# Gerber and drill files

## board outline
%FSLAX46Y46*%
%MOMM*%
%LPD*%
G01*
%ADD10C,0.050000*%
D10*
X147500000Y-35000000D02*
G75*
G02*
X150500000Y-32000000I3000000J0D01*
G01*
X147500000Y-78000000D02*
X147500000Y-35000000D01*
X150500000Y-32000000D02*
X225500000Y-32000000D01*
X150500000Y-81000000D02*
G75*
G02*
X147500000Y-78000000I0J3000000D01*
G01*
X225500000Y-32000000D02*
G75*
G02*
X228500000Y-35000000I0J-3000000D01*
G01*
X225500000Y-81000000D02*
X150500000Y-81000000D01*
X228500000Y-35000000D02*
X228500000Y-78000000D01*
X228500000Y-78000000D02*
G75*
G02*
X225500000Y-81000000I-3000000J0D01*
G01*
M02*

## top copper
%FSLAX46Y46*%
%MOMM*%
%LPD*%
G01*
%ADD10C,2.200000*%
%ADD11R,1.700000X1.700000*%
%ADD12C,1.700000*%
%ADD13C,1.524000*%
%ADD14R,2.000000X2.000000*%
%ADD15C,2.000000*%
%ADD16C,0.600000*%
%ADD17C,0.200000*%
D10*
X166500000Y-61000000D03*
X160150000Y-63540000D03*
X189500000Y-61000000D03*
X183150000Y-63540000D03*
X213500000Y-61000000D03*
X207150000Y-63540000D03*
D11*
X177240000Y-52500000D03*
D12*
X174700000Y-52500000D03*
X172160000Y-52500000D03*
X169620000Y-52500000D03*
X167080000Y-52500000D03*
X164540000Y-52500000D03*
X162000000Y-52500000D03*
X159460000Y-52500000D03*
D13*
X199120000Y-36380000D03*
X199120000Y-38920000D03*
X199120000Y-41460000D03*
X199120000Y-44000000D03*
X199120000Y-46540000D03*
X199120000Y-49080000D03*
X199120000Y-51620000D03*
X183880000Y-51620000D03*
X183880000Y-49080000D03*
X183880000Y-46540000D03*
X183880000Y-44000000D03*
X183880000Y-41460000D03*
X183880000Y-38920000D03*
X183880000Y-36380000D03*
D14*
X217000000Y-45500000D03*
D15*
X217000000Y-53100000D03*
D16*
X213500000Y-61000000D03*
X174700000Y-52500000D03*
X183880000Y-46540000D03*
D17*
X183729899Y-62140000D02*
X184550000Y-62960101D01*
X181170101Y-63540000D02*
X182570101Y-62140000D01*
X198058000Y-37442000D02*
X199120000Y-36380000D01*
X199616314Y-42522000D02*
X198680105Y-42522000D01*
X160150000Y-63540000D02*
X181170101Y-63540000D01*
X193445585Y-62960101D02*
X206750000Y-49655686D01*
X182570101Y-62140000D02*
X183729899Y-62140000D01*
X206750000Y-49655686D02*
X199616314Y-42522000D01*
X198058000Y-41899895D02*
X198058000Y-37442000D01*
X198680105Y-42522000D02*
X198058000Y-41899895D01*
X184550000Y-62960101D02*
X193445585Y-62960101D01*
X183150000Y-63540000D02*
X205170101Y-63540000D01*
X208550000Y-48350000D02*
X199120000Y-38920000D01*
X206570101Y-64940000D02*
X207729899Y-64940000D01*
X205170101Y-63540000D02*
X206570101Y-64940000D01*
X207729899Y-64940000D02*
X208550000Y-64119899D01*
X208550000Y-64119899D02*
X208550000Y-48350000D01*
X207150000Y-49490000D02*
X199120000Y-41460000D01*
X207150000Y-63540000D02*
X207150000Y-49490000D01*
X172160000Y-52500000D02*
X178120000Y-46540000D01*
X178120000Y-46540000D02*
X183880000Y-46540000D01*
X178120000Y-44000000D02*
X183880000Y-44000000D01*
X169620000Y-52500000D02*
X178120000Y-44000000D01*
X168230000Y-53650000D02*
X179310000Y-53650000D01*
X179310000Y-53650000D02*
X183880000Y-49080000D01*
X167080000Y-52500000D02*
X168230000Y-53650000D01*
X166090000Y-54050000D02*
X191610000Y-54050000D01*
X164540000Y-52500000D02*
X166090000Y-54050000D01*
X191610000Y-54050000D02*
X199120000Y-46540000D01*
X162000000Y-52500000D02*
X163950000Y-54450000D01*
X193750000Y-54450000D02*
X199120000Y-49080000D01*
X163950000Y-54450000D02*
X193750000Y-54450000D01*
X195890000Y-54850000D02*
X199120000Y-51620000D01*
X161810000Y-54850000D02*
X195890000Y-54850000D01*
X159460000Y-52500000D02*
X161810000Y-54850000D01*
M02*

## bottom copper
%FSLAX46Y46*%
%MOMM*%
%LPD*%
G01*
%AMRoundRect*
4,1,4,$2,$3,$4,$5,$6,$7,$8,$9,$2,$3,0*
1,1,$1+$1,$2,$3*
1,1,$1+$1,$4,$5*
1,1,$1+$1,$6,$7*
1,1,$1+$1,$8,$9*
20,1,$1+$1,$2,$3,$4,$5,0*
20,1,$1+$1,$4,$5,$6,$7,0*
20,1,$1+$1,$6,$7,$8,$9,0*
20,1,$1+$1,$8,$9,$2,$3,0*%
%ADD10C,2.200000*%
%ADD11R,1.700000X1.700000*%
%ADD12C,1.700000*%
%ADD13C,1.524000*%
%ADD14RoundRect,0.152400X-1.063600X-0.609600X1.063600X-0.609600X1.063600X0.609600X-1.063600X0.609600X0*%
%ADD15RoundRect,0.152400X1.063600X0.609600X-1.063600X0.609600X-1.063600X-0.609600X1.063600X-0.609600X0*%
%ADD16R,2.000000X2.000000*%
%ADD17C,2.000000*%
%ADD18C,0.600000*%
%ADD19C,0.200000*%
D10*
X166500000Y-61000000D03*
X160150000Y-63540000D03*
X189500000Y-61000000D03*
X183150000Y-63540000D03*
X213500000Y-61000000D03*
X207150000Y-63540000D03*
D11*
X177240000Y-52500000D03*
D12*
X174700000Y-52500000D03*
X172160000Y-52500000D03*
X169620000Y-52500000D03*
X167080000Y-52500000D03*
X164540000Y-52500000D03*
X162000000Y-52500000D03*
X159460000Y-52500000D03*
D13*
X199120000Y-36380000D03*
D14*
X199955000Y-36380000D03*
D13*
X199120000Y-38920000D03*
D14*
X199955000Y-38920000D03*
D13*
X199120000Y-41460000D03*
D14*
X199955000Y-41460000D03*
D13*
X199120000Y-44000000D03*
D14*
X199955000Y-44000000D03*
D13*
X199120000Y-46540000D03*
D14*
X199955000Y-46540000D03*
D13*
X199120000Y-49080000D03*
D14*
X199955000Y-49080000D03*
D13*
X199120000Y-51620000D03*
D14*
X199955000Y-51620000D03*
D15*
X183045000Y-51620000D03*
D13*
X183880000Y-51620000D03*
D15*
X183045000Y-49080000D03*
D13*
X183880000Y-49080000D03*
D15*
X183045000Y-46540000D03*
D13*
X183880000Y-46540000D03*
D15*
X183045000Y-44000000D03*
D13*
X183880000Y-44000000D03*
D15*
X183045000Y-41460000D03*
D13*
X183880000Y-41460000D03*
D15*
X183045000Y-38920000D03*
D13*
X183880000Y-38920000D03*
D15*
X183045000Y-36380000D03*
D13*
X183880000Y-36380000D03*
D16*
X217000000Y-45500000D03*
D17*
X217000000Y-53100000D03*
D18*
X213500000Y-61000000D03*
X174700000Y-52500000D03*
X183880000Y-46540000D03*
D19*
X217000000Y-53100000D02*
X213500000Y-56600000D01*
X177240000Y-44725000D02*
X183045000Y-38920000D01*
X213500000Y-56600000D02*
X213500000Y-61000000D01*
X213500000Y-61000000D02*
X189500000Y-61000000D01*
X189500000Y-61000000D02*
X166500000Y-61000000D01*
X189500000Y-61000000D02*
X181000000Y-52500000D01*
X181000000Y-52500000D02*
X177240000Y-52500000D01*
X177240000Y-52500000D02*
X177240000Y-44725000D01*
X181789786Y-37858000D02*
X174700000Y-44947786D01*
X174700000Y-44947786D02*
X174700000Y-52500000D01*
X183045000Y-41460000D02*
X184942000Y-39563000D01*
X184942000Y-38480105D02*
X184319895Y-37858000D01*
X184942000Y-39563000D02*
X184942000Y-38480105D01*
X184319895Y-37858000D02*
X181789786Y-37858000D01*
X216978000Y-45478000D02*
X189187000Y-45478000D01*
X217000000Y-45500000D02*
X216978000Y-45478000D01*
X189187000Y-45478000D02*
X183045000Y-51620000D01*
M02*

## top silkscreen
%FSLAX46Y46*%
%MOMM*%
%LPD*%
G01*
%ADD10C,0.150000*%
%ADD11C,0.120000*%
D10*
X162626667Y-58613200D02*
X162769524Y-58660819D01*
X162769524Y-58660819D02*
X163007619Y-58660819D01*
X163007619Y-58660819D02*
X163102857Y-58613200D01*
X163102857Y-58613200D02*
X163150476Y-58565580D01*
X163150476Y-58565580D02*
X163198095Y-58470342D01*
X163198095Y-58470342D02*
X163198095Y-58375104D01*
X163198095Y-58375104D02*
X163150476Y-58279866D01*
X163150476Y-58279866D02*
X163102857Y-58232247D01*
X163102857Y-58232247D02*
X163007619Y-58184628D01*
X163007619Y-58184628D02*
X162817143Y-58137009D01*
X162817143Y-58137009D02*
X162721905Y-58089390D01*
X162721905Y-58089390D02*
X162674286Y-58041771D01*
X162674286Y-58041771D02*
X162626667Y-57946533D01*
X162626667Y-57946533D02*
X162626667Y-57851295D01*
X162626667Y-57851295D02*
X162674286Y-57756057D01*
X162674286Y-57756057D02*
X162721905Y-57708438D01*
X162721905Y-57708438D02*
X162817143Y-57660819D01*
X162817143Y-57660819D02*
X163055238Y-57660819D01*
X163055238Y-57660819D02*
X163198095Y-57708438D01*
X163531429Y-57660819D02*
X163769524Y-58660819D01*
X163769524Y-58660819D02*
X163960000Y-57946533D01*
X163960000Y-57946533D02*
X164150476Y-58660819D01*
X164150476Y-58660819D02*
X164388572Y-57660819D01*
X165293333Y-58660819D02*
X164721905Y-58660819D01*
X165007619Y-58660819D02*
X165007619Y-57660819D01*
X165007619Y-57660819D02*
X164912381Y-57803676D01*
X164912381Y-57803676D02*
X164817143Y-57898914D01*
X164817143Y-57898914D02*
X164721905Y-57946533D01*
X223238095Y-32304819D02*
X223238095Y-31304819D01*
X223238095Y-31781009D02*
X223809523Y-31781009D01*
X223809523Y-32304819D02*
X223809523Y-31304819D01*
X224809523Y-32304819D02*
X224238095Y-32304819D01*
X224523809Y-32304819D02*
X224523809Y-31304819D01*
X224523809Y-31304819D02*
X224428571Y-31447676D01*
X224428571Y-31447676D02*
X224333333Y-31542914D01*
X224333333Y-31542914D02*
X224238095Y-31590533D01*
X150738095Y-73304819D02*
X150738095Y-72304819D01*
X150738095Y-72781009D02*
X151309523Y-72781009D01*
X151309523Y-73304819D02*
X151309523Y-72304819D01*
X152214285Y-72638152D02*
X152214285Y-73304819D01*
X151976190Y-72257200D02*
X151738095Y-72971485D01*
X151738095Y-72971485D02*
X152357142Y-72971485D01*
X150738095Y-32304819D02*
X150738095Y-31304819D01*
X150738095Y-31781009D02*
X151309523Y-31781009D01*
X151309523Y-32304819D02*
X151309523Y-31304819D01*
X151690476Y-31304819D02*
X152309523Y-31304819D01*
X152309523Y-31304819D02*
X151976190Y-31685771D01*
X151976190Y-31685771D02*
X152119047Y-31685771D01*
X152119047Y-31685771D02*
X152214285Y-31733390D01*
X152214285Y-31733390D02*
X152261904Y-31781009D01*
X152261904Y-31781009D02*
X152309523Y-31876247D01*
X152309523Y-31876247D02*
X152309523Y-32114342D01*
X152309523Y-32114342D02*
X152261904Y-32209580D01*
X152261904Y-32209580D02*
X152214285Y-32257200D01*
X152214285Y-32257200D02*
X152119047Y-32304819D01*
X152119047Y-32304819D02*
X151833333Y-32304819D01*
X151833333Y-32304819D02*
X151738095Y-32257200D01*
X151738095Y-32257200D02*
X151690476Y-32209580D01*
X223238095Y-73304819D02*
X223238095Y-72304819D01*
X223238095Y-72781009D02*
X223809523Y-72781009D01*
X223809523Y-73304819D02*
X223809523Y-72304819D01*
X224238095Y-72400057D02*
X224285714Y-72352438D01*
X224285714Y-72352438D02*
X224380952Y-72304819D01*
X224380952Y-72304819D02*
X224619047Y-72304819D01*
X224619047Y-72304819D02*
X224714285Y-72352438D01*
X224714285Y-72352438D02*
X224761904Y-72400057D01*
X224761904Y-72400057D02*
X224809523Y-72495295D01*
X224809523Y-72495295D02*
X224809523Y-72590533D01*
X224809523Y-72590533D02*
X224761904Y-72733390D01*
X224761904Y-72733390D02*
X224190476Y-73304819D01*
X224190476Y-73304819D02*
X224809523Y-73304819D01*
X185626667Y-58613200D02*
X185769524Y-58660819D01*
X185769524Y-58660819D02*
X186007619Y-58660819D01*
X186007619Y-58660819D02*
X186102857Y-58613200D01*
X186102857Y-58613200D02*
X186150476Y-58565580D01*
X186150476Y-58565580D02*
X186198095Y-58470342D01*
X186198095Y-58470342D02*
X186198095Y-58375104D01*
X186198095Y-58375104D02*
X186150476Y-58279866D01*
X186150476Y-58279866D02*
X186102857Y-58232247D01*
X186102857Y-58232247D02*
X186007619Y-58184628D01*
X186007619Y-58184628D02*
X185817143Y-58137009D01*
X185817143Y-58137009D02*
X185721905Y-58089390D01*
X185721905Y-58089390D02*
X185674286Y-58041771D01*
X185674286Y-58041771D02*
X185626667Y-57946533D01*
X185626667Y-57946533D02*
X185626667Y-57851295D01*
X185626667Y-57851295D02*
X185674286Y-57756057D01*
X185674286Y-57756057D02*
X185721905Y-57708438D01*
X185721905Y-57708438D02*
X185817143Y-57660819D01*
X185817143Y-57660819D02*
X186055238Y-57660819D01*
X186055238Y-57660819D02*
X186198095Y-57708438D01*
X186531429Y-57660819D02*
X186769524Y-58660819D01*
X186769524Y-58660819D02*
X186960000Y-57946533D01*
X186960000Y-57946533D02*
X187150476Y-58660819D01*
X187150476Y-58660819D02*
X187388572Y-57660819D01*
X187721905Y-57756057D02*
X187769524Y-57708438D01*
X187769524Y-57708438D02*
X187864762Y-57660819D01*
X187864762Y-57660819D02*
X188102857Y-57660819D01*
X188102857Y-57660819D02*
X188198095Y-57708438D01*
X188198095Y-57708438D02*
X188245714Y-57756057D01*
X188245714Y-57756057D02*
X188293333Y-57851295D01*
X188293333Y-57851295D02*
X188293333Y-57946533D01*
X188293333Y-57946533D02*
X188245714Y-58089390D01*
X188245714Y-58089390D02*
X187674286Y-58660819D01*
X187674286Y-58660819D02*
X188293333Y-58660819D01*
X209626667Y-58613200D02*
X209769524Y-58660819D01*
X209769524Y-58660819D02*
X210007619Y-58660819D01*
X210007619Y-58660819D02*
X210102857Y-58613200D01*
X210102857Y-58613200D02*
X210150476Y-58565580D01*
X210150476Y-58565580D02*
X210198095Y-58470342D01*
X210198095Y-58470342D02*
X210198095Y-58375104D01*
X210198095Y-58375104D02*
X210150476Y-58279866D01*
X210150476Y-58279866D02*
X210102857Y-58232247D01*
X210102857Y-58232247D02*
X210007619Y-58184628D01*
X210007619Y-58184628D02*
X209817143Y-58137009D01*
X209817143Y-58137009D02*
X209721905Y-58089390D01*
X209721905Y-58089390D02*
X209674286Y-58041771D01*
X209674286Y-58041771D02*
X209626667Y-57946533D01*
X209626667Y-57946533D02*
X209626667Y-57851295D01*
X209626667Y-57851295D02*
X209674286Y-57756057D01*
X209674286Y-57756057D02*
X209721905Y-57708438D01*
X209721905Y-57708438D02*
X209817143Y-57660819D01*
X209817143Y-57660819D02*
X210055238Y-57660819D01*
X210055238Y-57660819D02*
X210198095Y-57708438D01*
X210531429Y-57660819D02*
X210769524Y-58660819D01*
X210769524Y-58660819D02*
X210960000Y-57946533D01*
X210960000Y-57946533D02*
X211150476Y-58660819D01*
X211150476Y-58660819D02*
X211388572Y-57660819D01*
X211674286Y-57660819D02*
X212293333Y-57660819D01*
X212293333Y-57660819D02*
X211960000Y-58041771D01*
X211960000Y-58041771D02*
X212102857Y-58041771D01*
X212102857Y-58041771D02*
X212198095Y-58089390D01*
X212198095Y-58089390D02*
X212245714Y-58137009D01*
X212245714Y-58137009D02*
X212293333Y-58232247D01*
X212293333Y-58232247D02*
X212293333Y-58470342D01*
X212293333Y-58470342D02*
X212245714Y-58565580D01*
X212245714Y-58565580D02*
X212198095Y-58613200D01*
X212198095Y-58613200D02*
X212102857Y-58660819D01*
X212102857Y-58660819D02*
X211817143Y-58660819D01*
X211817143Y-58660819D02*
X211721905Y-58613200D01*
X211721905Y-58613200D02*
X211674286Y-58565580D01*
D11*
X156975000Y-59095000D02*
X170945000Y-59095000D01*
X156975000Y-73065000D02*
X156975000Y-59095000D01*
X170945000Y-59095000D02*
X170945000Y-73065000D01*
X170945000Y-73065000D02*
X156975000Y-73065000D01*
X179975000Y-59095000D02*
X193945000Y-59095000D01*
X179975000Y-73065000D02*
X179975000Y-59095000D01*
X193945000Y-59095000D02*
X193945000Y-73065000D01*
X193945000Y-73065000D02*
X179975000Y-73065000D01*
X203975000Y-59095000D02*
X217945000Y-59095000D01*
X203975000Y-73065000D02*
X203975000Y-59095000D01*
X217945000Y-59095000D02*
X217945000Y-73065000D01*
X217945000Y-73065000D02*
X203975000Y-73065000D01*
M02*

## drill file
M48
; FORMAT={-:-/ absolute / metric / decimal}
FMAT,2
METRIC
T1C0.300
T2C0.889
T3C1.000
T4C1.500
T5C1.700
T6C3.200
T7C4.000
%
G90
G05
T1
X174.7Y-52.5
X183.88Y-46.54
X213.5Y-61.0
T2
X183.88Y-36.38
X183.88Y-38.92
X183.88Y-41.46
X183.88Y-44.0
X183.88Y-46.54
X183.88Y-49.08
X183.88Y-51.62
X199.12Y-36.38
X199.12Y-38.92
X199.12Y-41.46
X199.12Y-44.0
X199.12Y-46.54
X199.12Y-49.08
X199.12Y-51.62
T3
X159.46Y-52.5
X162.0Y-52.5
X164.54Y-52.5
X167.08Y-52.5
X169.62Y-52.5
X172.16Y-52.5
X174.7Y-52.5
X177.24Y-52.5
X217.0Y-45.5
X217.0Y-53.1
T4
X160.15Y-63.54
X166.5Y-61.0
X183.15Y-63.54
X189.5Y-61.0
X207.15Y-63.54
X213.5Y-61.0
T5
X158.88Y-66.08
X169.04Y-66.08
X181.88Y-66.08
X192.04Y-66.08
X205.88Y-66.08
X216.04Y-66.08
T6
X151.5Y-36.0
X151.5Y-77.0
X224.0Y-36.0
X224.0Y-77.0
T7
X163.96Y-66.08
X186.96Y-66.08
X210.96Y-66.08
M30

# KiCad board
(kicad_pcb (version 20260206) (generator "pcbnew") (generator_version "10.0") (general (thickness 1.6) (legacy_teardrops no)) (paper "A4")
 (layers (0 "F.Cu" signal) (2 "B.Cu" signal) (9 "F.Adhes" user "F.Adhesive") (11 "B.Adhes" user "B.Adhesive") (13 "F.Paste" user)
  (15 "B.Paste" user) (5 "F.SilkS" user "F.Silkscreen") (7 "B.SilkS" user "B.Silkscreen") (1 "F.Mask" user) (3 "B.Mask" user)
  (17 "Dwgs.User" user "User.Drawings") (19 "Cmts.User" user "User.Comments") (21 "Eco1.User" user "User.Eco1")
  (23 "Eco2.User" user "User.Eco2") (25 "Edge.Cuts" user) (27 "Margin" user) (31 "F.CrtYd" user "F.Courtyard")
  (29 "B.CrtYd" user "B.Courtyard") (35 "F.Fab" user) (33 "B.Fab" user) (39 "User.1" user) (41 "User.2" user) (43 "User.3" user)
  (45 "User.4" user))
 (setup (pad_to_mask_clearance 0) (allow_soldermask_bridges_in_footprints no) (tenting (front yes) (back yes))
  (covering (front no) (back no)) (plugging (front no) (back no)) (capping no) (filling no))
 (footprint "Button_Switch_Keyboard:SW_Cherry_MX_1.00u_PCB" (layer "F.Cu") (at 166.5 61)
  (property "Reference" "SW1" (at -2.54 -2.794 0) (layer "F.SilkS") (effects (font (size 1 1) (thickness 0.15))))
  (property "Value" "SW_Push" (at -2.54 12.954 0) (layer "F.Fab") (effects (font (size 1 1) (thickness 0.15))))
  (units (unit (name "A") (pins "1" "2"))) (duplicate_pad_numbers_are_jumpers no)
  (fp_line (start -9.525 -1.905) (end 4.445 -1.905) (stroke (width 0.12) (type solid)) (layer "F.SilkS"))
  (fp_line (start -9.525 12.065) (end -9.525 -1.905) (stroke (width 0.12) (type solid)) (layer "F.SilkS"))
  (fp_line (start 4.445 -1.905) (end 4.445 12.065) (stroke (width 0.12) (type solid)) (layer "F.SilkS"))
  (fp_line (start 4.445 12.065) (end -9.525 12.065) (stroke (width 0.12) (type solid)) (layer "F.SilkS"))
  (pad "" np_thru_hole circle (at -7.62 5.08) (size 1.7 1.7) (drill 1.7) (layers "*.Cu" "*.Mask"))
  (pad "" np_thru_hole circle (at -2.54 5.08) (size 4 4) (drill 4) (layers "*.Cu" "*.Mask"))
  (pad "" np_thru_hole circle (at 2.54 5.08) (size 1.7 1.7) (drill 1.7) (layers "*.Cu" "*.Mask"))
  (pad "1" thru_hole circle (at 0 0) (size 2.2 2.2) (drill 1.5) (layers "*.Cu" "*.Mask") (remove_unused_layers no) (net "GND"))
  (pad "2" thru_hole circle (at -6.35 2.54) (size 2.2 2.2) (drill 1.5) (layers "*.Cu" "*.Mask") (remove_unused_layers no)
   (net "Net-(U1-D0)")))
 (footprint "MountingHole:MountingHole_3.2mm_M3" (layer "F.Cu") (at 224 36)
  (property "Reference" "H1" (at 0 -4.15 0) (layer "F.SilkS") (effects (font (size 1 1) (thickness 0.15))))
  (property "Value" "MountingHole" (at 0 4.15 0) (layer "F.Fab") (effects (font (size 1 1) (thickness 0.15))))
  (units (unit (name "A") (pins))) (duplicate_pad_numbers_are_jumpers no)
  (pad "" np_thru_hole circle (at 0 0) (size 3.2 3.2) (drill 3.2) (layers "*.Cu" "*.Mask")))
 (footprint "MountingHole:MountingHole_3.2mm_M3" (layer "F.Cu") (at 151.5 77)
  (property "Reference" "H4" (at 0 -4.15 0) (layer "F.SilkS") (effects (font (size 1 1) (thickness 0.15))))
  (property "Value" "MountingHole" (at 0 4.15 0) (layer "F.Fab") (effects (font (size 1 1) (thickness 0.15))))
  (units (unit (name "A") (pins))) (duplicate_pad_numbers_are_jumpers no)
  (pad "" np_thru_hole circle (at 0 0) (size 3.2 3.2) (drill 3.2) (layers "*.Cu" "*.Mask")))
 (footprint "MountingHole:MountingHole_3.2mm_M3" (layer "F.Cu") (at 151.5 36)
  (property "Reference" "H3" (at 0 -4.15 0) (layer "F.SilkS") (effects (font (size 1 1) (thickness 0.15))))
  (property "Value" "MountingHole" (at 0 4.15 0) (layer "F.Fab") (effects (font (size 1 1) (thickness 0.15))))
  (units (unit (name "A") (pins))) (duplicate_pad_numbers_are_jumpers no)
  (pad "" np_thru_hole circle (at 0 0) (size 3.2 3.2) (drill 3.2) (layers "*.Cu" "*.Mask")))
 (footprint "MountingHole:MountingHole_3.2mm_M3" (layer "F.Cu") (at 224 77)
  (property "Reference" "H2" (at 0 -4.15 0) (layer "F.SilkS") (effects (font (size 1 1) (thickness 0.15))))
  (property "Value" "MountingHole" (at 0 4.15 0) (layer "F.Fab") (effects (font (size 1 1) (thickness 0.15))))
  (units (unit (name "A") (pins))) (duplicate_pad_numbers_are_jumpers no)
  (pad "" np_thru_hole circle (at 0 0) (size 3.2 3.2) (drill 3.2) (layers "*.Cu" "*.Mask")))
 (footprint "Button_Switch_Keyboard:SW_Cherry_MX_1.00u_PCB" (layer "F.Cu") (at 189.5 61)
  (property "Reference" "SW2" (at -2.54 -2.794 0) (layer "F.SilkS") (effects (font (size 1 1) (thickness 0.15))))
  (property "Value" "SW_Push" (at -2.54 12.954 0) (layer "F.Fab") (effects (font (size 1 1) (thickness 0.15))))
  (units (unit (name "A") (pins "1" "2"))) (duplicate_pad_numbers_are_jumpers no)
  (fp_line (start -9.525 -1.905) (end 4.445 -1.905) (stroke (width 0.12) (type solid)) (layer "F.SilkS"))
  (fp_line (start -9.525 12.065) (end -9.525 -1.905) (stroke (width 0.12) (type solid)) (layer "F.SilkS"))
  (fp_line (start 4.445 -1.905) (end 4.445 12.065) (stroke (width 0.12) (type solid)) (layer "F.SilkS"))
  (fp_line (start 4.445 12.065) (end -9.525 12.065) (stroke (width 0.12) (type solid)) (layer "F.SilkS"))
  (pad "" np_thru_hole circle (at -7.62 5.08) (size 1.7 1.7) (drill 1.7) (layers "*.Cu" "*.Mask"))
  (pad "" np_thru_hole circle (at -2.54 5.08) (size 4 4) (drill 4) (layers "*.Cu" "*.Mask"))
  (pad "" np_thru_hole circle (at 2.54 5.08) (size 1.7 1.7) (drill 1.7) (layers "*.Cu" "*.Mask"))
  (pad "1" thru_hole circle (at 0 0) (size 2.2 2.2) (drill 1.5) (layers "*.Cu" "*.Mask") (remove_unused_layers no) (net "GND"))
  (pad "2" thru_hole circle (at -6.35 2.54) (size 2.2 2.2) (drill 1.5) (layers "*.Cu" "*.Mask") (remove_unused_layers no)
   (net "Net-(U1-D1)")))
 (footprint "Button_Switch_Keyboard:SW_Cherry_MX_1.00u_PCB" (layer "F.Cu") (at 213.5 61)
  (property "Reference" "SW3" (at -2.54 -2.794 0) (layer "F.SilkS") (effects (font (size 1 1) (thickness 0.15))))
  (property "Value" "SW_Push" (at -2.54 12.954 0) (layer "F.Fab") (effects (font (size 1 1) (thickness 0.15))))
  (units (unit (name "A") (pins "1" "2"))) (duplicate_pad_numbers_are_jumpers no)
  (fp_line (start -9.525 -1.905) (end 4.445 -1.905) (stroke (width 0.12) (type solid)) (layer "F.SilkS"))
  (fp_line (start -9.525 12.065) (end -9.525 -1.905) (stroke (width 0.12) (type solid)) (layer "F.SilkS"))
  (fp_line (start 4.445 -1.905) (end 4.445 12.065) (stroke (width 0.12) (type solid)) (layer "F.SilkS"))
  (fp_line (start 4.445 12.065) (end -9.525 12.065) (stroke (width 0.12) (type solid)) (layer "F.SilkS"))
  (pad "" np_thru_hole circle (at -7.62 5.08) (size 1.7 1.7) (drill 1.7) (layers "*.Cu" "*.Mask"))
  (pad "" np_thru_hole circle (at -2.54 5.08) (size 4 4) (drill 4) (layers "*.Cu" "*.Mask"))
  (pad "" np_thru_hole circle (at 2.54 5.08) (size 1.7 1.7) (drill 1.7) (layers "*.Cu" "*.Mask"))
  (pad "1" thru_hole circle (at 0 0) (size 2.2 2.2) (drill 1.5) (layers "*.Cu" "*.Mask") (remove_unused_layers no) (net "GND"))
  (pad "2" thru_hole circle (at -6.35 2.54) (size 2.2 2.2) (drill 1.5) (layers "*.Cu" "*.Mask") (remove_unused_layers no)
   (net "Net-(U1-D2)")))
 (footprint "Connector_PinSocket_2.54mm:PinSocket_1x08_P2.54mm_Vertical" (layer "B.Cu") (at 177.24 52.5 90)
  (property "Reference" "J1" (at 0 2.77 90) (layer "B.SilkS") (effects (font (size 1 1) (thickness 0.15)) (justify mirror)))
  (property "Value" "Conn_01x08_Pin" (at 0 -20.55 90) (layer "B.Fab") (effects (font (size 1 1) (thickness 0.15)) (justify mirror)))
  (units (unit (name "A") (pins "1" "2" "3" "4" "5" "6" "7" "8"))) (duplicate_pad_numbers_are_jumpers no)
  (pad "1" thru_hole rect (at 0 0 90) (size 1.7 1.7) (drill 1) (layers "*.Cu" "*.Mask") (remove_unused_layers no) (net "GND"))
  (pad "2" thru_hole circle (at 0 -2.54 90) (size 1.7 1.7) (drill 1) (layers "*.Cu" "*.Mask") (remove_unused_layers no) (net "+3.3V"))
  (pad "3" thru_hole circle (at 0 -5.08 90) (size 1.7 1.7) (drill 1) (layers "*.Cu" "*.Mask") (remove_unused_layers no) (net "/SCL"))
  (pad "4" thru_hole circle (at 0 -7.62 90) (size 1.7 1.7) (drill 1) (layers "*.Cu" "*.Mask") (remove_unused_layers no) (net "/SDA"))
  (pad "5" thru_hole circle (at 0 -10.16 90) (size 1.7 1.7) (drill 1) (layers "*.Cu" "*.Mask") (remove_unused_layers no) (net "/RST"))
  (pad "6" thru_hole circle (at 0 -12.7 90) (size 1.7 1.7) (drill 1) (layers "*.Cu" "*.Mask") (remove_unused_layers no) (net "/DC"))
  (pad "7" thru_hole circle (at 0 -15.24 90) (size 1.7 1.7) (drill 1) (layers "*.Cu" "*.Mask") (remove_unused_layers no) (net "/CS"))
  (pad "8" thru_hole circle (at 0 -17.78 90) (size 1.7 1.7) (drill 1) (layers "*.Cu" "*.Mask") (remove_unused_layers no) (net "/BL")))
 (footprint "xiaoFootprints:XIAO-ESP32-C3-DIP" (layer "B.Cu") (at 191.5 44 90)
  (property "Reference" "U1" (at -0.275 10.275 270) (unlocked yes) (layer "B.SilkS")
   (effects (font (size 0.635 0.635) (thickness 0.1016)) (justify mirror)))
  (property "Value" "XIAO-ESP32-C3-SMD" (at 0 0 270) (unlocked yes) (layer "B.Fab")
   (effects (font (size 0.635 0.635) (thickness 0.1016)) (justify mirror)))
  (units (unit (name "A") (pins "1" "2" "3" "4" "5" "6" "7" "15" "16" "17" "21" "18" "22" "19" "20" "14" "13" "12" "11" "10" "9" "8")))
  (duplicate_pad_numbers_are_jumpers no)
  (pad "1" thru_hole circle (at 7.62 7.62) (size 1.524 1.524) (drill 0.889) (layers "*.Cu" "*.Mask") (remove_unused_layers no)
   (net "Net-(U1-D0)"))
  (pad "1" smd roundrect (at 7.62 8.455) (size 2.432 1.524) (layers "B.Cu" "B.Mask") (roundrect_rratio 0.1) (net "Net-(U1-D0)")
   (thermal_bridge_angle 45))
  (pad "2" thru_hole circle (at 5.08 7.62) (size 1.524 1.524) (drill 0.889) (layers "*.Cu" "*.Mask") (remove_unused_layers no)
   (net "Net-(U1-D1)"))
  (pad "2" smd roundrect (at 5.08 8.455) (size 2.432 1.524) (layers "B.Cu" "B.Mask") (roundrect_rratio 0.1) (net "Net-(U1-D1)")
   (thermal_bridge_angle 45))
  (pad "3" thru_hole circle (at 2.54 7.62) (size 1.524 1.524) (drill 0.889) (layers "*.Cu" "*.Mask") (remove_unused_layers no)
   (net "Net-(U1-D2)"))
  (pad "3" smd roundrect (at 2.54 8.455) (size 2.432 1.524) (layers "B.Cu" "B.Mask") (roundrect_rratio 0.1) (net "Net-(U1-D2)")
   (thermal_bridge_angle 45))
  (pad "4" thru_hole circle (at 0 7.62) (size 1.524 1.524) (drill 0.889) (layers "*.Cu" "*.Mask") (remove_unused_layers no)
   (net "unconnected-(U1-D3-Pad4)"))
  (pad "4" smd roundrect (at 0 8.455) (size 2.432 1.524) (layers "B.Cu" "B.Mask") (roundrect_rratio 0.1) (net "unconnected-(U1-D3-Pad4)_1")
   (thermal_bridge_angle 45))
  (pad "5" thru_hole circle (at -2.54 7.62) (size 1.524 1.524) (drill 0.889) (layers "*.Cu" "*.Mask") (remove_unused_layers no) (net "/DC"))
  (pad "5" smd roundrect (at -2.54 8.455) (size 2.432 1.524) (layers "B.Cu" "B.Mask") (roundrect_rratio 0.1) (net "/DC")
   (thermal_bridge_angle 45))
  (pad "6" thru_hole circle (at -5.08 7.62) (size 1.524 1.524) (drill 0.889) (layers "*.Cu" "*.Mask") (remove_unused_layers no) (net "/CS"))
  (pad "6" smd roundrect (at -5.08 8.455) (size 2.432 1.524) (layers "B.Cu" "B.Mask") (roundrect_rratio 0.1) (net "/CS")
   (thermal_bridge_angle 45))
  (pad "7" thru_hole circle (at -7.62 7.62) (size 1.524 1.524) (drill 0.889) (layers "*.Cu" "*.Mask") (remove_unused_layers no) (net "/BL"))
  (pad "7" smd roundrect (at -7.62 8.455) (size 2.432 1.524) (layers "B.Cu" "B.Mask") (roundrect_rratio 0.1) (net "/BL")
   (thermal_bridge_angle 45))
  (pad "8" smd roundrect (at -7.62 -8.455 180) (size 2.432 1.524) (layers "B.Cu" "B.Mask") (roundrect_rratio 0.1) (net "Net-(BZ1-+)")
   (thermal_bridge_angle 45))
  (pad "8" thru_hole circle (at -7.62 -7.62 180) (size 1.524 1.524) (drill 0.889) (layers "*.Cu" "*.Mask") (remove_unused_layers no)
   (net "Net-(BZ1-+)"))
  (pad "9" smd roundrect (at -5.08 -8.455 180) (size 2.432 1.524) (layers "B.Cu" "B.Mask") (roundrect_rratio 0.1) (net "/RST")
   (thermal_bridge_angle 45))
  (pad "9" thru_hole circle (at -5.08 -7.62 180) (size 1.524 1.524) (drill 0.889) (layers "*.Cu" "*.Mask") (remove_unused_layers no)
   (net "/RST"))
  (pad "10" smd roundrect (at -2.54 -8.455 180) (size 2.432 1.524) (layers "B.Cu" "B.Mask") (roundrect_rratio 0.1) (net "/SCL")
   (thermal_bridge_angle 45))
  (pad "10" thru_hole circle (at -2.54 -7.62 180) (size 1.524 1.524) (drill 0.889) (layers "*.Cu" "*.Mask") (remove_unused_layers no)
   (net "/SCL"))
  (pad "11" smd roundrect (at 0 -8.455 180) (size 2.432 1.524) (layers "B.Cu" "B.Mask") (roundrect_rratio 0.1) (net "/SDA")
   (thermal_bridge_angle 45))
  (pad "11" thru_hole circle (at 0 -7.62 180) (size 1.524 1.524) (drill 0.889) (layers "*.Cu" "*.Mask") (remove_unused_layers no)
   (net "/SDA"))
  (pad "12" smd roundrect (at 2.54 -8.455 180) (size 2.432 1.524) (layers "B.Cu" "B.Mask") (roundrect_rratio 0.1) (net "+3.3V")
   (thermal_bridge_angle 45))
  (pad "12" thru_hole circle (at 2.54 -7.62 180) (size 1.524 1.524) (drill 0.889) (layers "*.Cu" "*.Mask") (remove_unused_layers no)
   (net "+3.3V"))
  (pad "13" smd roundrect (at 5.08 -8.455 180) (size 2.432 1.524) (layers "B.Cu" "B.Mask") (roundrect_rratio 0.1) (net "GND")
   (thermal_bridge_angle 45))
  (pad "13" thru_hole circle (at 5.08 -7.62 180) (size 1.524 1.524) (drill 0.889) (layers "*.Cu" "*.Mask") (remove_unused_layers no)
   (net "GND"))
  (pad "14" smd roundrect (at 7.62 -8.455 180) (size 2.432 1.524) (layers "B.Cu" "B.Mask") (roundrect_rratio 0.1)
   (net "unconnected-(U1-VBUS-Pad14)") (thermal_bridge_angle 45))
  (pad "14" thru_hole circle (at 7.62 -7.62 180) (size 1.524 1.524) (drill 0.889) (layers "*.Cu" "*.Mask") (remove_unused_layers no)
   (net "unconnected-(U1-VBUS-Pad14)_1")))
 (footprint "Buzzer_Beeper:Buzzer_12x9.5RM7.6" (layer "B.Cu") (at 217 45.5 -90)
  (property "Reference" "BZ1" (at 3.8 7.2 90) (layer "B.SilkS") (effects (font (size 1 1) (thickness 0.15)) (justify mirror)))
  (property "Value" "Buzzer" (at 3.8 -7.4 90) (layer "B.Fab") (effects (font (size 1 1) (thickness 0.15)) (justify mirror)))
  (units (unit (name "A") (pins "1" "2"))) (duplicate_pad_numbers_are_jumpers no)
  (pad "1" thru_hole rect (at 0 0 270) (size 2 2) (drill 1) (layers "*.Cu" "*.Mask") (remove_unused_layers no) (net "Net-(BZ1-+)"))
  (pad "2" thru_hole circle (at 7.6 0 270) (size 2 2) (drill 1) (layers "*.Cu" "*.Mask") (remove_unused_layers no) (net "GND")))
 (gr_arc (start 147.5 35) (mid 148.37868 32.87868) (end 150.5 32) (stroke (width 0.05) (type default)) (layer "Edge.Cuts"))
 (gr_line (start 147.5 78) (end 147.5 35) (stroke (width 0.05) (type default)) (layer "Edge.Cuts"))
 (gr_line (start 150.5 32) (end 225.5 32) (stroke (width 0.05) (type default)) (layer "Edge.Cuts"))
 (gr_arc (start 150.5 81) (mid 148.37868 80.12132) (end 147.5 78) (stroke (width 0.05) (type default)) (layer "Edge.Cuts"))
 (gr_arc (start 225.5 32) (mid 227.62132 32.87868) (end 228.5 35) (stroke (width 0.05) (type default)) (layer "Edge.Cuts"))
 (gr_line (start 225.5 81) (end 150.5 81) (stroke (width 0.05) (type default)) (layer "Edge.Cuts"))
 (gr_line (start 228.5 35) (end 228.5 78) (stroke (width 0.05) (type default)) (layer "Edge.Cuts"))
 (gr_arc (start 228.5 78) (mid 227.62132 80.12132) (end 225.5 81) (stroke (width 0.05) (type default)) (layer "Edge.Cuts"))
 (via (at 213.5 61) (size 0.6) (drill 0.3) (layers "F.Cu" "B.Cu") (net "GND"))
 (segment (start 217 53.1) (end 213.5 56.6) (width 0.2) (layer "B.Cu") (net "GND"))
 (segment (start 177.24 44.725) (end 183.045 38.92) (width 0.2) (layer "B.Cu") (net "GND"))
 (segment (start 213.5 56.6) (end 213.5 61) (width 0.2) (layer "B.Cu") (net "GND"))
 (segment (start 213.5 61) (end 189.5 61) (width 0.2) (layer "B.Cu") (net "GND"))
 (segment (start 189.5 61) (end 166.5 61) (width 0.2) (layer "B.Cu") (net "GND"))
 (segment (start 189.5 61) (end 181 52.5) (width 0.2) (layer "B.Cu") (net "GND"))
 (segment (start 181 52.5) (end 177.24 52.5) (width 0.2) (layer "B.Cu") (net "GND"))
 (segment (start 177.24 52.5) (end 177.24 44.725) (width 0.2) (layer "B.Cu") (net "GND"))
 (segment (start 183.729899 62.14) (end 184.55 62.960101) (width 0.2) (layer "F.Cu") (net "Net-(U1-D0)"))
 (segment (start 181.170101 63.54) (end 182.570101 62.14) (width 0.2) (layer "F.Cu") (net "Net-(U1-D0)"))
 (segment (start 198.058 37.442) (end 199.12 36.38) (width 0.2) (layer "F.Cu") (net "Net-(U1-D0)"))
 (segment (start 199.616314 42.522) (end 198.680105 42.522) (width 0.2) (layer "F.Cu") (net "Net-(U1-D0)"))
 (segment (start 160.15 63.54) (end 181.170101 63.54) (width 0.2) (layer "F.Cu") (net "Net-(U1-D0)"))
 (segment (start 193.445585 62.960101) (end 206.75 49.655686) (width 0.2) (layer "F.Cu") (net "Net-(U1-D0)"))
 (segment (start 182.570101 62.14) (end 183.729899 62.14) (width 0.2) (layer "F.Cu") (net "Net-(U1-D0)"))
 (segment (start 206.75 49.655686) (end 199.616314 42.522) (width 0.2) (layer "F.Cu") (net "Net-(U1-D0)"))
 (segment (start 198.058 41.899895) (end 198.058 37.442) (width 0.2) (layer "F.Cu") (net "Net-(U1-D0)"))
 (segment (start 198.680105 42.522) (end 198.058 41.899895) (width 0.2) (layer "F.Cu") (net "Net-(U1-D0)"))
 (segment (start 184.55 62.960101) (end 193.445585 62.960101) (width 0.2) (layer "F.Cu") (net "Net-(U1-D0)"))
 (segment (start 183.15 63.54) (end 205.170101 63.54) (width 0.2) (layer "F.Cu") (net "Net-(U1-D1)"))
 (segment (start 208.55 48.35) (end 199.12 38.92) (width 0.2) (layer "F.Cu") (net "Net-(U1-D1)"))
 (segment (start 206.570101 64.94) (end 207.729899 64.94) (width 0.2) (layer "F.Cu") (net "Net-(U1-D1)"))
 (segment (start 205.170101 63.54) (end 206.570101 64.94) (width 0.2) (layer "F.Cu") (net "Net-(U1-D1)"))
 (segment (start 207.729899 64.94) (end 208.55 64.119899) (width 0.2) (layer "F.Cu") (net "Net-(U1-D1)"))
 (segment (start 208.55 64.119899) (end 208.55 48.35) (width 0.2) (layer "F.Cu") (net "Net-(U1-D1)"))
 (segment (start 207.15 49.49) (end 199.12 41.46) (width 0.2) (layer "F.Cu") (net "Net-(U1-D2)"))
 (segment (start 207.15 63.54) (end 207.15 49.49) (width 0.2) (layer "F.Cu") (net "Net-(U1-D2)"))
 (via (at 174.7 52.5) (size 0.6) (drill 0.3) (layers "F.Cu" "B.Cu") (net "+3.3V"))
 (segment (start 181.789786 37.858) (end 174.7 44.947786) (width 0.2) (layer "B.Cu") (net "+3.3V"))
 (segment (start 174.7 44.947786) (end 174.7 52.5) (width 0.2) (layer "B.Cu") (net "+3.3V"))
 (segment (start 183.045 41.46) (end 184.942 39.563) (width 0.2) (layer "B.Cu") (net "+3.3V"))
 (segment (start 184.942 38.480105) (end 184.319895 37.858) (width 0.2) (layer "B.Cu") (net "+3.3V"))
 (segment (start 184.942 39.563) (end 184.942 38.480105) (width 0.2) (layer "B.Cu") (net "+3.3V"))
 (segment (start 184.319895 37.858) (end 181.789786 37.858) (width 0.2) (layer "B.Cu") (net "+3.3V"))
 (segment (start 172.16 52.5) (end 178.12 46.54) (width 0.2) (layer "F.Cu") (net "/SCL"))
 (segment (start 178.12 46.54) (end 183.88 46.54) (width 0.2) (layer "F.Cu") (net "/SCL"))
 (via (at 183.88 46.54) (size 0.6) (drill 0.3) (layers "F.Cu" "B.Cu") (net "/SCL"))
 (segment (start 178.12 44) (end 183.88 44) (width 0.2) (layer "F.Cu") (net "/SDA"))
 (segment (start 169.62 52.5) (end 178.12 44) (width 0.2) (layer "F.Cu") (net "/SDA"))
 (segment (start 168.23 53.65) (end 179.31 53.65) (width 0.2) (layer "F.Cu") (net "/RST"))
 (segment (start 179.31 53.65) (end 183.88 49.08) (width 0.2) (layer "F.Cu") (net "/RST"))
 (segment (start 167.08 52.5) (end 168.23 53.65) (width 0.2) (layer "F.Cu") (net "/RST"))
 (segment (start 166.09 54.05) (end 191.61 54.05) (width 0.2) (layer "F.Cu") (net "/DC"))
 (segment (start 164.54 52.5) (end 166.09 54.05) (width 0.2) (layer "F.Cu") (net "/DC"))
 (segment (start 191.61 54.05) (end 199.12 46.54) (width 0.2) (layer "F.Cu") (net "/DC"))
 (segment (start 162 52.5) (end 163.95 54.45) (width 0.2) (layer "F.Cu") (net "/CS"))
 (segment (start 193.75 54.45) (end 199.12 49.08) (width 0.2) (layer "F.Cu") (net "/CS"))
 (segment (start 163.95 54.45) (end 193.75 54.45) (width 0.2) (layer "F.Cu") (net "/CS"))
 (segment (start 195.89 54.85) (end 199.12 51.62) (width 0.2) (layer "F.Cu") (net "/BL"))
 (segment (start 161.81 54.85) (end 195.89 54.85) (width 0.2) (layer "F.Cu") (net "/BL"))
 (segment (start 159.46 52.5) (end 161.81 54.85) (width 0.2) (layer "F.Cu") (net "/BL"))
 (segment (start 216.978 45.478) (end 189.187 45.478) (width 0.2) (layer "B.Cu") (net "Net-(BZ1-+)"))
 (segment (start 217 45.5) (end 216.978 45.478) (width 0.2) (layer "B.Cu") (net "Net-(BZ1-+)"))
 (segment (start 189.187 45.478) (end 183.045 51.62) (width 0.2) (layer "B.Cu") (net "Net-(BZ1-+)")))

